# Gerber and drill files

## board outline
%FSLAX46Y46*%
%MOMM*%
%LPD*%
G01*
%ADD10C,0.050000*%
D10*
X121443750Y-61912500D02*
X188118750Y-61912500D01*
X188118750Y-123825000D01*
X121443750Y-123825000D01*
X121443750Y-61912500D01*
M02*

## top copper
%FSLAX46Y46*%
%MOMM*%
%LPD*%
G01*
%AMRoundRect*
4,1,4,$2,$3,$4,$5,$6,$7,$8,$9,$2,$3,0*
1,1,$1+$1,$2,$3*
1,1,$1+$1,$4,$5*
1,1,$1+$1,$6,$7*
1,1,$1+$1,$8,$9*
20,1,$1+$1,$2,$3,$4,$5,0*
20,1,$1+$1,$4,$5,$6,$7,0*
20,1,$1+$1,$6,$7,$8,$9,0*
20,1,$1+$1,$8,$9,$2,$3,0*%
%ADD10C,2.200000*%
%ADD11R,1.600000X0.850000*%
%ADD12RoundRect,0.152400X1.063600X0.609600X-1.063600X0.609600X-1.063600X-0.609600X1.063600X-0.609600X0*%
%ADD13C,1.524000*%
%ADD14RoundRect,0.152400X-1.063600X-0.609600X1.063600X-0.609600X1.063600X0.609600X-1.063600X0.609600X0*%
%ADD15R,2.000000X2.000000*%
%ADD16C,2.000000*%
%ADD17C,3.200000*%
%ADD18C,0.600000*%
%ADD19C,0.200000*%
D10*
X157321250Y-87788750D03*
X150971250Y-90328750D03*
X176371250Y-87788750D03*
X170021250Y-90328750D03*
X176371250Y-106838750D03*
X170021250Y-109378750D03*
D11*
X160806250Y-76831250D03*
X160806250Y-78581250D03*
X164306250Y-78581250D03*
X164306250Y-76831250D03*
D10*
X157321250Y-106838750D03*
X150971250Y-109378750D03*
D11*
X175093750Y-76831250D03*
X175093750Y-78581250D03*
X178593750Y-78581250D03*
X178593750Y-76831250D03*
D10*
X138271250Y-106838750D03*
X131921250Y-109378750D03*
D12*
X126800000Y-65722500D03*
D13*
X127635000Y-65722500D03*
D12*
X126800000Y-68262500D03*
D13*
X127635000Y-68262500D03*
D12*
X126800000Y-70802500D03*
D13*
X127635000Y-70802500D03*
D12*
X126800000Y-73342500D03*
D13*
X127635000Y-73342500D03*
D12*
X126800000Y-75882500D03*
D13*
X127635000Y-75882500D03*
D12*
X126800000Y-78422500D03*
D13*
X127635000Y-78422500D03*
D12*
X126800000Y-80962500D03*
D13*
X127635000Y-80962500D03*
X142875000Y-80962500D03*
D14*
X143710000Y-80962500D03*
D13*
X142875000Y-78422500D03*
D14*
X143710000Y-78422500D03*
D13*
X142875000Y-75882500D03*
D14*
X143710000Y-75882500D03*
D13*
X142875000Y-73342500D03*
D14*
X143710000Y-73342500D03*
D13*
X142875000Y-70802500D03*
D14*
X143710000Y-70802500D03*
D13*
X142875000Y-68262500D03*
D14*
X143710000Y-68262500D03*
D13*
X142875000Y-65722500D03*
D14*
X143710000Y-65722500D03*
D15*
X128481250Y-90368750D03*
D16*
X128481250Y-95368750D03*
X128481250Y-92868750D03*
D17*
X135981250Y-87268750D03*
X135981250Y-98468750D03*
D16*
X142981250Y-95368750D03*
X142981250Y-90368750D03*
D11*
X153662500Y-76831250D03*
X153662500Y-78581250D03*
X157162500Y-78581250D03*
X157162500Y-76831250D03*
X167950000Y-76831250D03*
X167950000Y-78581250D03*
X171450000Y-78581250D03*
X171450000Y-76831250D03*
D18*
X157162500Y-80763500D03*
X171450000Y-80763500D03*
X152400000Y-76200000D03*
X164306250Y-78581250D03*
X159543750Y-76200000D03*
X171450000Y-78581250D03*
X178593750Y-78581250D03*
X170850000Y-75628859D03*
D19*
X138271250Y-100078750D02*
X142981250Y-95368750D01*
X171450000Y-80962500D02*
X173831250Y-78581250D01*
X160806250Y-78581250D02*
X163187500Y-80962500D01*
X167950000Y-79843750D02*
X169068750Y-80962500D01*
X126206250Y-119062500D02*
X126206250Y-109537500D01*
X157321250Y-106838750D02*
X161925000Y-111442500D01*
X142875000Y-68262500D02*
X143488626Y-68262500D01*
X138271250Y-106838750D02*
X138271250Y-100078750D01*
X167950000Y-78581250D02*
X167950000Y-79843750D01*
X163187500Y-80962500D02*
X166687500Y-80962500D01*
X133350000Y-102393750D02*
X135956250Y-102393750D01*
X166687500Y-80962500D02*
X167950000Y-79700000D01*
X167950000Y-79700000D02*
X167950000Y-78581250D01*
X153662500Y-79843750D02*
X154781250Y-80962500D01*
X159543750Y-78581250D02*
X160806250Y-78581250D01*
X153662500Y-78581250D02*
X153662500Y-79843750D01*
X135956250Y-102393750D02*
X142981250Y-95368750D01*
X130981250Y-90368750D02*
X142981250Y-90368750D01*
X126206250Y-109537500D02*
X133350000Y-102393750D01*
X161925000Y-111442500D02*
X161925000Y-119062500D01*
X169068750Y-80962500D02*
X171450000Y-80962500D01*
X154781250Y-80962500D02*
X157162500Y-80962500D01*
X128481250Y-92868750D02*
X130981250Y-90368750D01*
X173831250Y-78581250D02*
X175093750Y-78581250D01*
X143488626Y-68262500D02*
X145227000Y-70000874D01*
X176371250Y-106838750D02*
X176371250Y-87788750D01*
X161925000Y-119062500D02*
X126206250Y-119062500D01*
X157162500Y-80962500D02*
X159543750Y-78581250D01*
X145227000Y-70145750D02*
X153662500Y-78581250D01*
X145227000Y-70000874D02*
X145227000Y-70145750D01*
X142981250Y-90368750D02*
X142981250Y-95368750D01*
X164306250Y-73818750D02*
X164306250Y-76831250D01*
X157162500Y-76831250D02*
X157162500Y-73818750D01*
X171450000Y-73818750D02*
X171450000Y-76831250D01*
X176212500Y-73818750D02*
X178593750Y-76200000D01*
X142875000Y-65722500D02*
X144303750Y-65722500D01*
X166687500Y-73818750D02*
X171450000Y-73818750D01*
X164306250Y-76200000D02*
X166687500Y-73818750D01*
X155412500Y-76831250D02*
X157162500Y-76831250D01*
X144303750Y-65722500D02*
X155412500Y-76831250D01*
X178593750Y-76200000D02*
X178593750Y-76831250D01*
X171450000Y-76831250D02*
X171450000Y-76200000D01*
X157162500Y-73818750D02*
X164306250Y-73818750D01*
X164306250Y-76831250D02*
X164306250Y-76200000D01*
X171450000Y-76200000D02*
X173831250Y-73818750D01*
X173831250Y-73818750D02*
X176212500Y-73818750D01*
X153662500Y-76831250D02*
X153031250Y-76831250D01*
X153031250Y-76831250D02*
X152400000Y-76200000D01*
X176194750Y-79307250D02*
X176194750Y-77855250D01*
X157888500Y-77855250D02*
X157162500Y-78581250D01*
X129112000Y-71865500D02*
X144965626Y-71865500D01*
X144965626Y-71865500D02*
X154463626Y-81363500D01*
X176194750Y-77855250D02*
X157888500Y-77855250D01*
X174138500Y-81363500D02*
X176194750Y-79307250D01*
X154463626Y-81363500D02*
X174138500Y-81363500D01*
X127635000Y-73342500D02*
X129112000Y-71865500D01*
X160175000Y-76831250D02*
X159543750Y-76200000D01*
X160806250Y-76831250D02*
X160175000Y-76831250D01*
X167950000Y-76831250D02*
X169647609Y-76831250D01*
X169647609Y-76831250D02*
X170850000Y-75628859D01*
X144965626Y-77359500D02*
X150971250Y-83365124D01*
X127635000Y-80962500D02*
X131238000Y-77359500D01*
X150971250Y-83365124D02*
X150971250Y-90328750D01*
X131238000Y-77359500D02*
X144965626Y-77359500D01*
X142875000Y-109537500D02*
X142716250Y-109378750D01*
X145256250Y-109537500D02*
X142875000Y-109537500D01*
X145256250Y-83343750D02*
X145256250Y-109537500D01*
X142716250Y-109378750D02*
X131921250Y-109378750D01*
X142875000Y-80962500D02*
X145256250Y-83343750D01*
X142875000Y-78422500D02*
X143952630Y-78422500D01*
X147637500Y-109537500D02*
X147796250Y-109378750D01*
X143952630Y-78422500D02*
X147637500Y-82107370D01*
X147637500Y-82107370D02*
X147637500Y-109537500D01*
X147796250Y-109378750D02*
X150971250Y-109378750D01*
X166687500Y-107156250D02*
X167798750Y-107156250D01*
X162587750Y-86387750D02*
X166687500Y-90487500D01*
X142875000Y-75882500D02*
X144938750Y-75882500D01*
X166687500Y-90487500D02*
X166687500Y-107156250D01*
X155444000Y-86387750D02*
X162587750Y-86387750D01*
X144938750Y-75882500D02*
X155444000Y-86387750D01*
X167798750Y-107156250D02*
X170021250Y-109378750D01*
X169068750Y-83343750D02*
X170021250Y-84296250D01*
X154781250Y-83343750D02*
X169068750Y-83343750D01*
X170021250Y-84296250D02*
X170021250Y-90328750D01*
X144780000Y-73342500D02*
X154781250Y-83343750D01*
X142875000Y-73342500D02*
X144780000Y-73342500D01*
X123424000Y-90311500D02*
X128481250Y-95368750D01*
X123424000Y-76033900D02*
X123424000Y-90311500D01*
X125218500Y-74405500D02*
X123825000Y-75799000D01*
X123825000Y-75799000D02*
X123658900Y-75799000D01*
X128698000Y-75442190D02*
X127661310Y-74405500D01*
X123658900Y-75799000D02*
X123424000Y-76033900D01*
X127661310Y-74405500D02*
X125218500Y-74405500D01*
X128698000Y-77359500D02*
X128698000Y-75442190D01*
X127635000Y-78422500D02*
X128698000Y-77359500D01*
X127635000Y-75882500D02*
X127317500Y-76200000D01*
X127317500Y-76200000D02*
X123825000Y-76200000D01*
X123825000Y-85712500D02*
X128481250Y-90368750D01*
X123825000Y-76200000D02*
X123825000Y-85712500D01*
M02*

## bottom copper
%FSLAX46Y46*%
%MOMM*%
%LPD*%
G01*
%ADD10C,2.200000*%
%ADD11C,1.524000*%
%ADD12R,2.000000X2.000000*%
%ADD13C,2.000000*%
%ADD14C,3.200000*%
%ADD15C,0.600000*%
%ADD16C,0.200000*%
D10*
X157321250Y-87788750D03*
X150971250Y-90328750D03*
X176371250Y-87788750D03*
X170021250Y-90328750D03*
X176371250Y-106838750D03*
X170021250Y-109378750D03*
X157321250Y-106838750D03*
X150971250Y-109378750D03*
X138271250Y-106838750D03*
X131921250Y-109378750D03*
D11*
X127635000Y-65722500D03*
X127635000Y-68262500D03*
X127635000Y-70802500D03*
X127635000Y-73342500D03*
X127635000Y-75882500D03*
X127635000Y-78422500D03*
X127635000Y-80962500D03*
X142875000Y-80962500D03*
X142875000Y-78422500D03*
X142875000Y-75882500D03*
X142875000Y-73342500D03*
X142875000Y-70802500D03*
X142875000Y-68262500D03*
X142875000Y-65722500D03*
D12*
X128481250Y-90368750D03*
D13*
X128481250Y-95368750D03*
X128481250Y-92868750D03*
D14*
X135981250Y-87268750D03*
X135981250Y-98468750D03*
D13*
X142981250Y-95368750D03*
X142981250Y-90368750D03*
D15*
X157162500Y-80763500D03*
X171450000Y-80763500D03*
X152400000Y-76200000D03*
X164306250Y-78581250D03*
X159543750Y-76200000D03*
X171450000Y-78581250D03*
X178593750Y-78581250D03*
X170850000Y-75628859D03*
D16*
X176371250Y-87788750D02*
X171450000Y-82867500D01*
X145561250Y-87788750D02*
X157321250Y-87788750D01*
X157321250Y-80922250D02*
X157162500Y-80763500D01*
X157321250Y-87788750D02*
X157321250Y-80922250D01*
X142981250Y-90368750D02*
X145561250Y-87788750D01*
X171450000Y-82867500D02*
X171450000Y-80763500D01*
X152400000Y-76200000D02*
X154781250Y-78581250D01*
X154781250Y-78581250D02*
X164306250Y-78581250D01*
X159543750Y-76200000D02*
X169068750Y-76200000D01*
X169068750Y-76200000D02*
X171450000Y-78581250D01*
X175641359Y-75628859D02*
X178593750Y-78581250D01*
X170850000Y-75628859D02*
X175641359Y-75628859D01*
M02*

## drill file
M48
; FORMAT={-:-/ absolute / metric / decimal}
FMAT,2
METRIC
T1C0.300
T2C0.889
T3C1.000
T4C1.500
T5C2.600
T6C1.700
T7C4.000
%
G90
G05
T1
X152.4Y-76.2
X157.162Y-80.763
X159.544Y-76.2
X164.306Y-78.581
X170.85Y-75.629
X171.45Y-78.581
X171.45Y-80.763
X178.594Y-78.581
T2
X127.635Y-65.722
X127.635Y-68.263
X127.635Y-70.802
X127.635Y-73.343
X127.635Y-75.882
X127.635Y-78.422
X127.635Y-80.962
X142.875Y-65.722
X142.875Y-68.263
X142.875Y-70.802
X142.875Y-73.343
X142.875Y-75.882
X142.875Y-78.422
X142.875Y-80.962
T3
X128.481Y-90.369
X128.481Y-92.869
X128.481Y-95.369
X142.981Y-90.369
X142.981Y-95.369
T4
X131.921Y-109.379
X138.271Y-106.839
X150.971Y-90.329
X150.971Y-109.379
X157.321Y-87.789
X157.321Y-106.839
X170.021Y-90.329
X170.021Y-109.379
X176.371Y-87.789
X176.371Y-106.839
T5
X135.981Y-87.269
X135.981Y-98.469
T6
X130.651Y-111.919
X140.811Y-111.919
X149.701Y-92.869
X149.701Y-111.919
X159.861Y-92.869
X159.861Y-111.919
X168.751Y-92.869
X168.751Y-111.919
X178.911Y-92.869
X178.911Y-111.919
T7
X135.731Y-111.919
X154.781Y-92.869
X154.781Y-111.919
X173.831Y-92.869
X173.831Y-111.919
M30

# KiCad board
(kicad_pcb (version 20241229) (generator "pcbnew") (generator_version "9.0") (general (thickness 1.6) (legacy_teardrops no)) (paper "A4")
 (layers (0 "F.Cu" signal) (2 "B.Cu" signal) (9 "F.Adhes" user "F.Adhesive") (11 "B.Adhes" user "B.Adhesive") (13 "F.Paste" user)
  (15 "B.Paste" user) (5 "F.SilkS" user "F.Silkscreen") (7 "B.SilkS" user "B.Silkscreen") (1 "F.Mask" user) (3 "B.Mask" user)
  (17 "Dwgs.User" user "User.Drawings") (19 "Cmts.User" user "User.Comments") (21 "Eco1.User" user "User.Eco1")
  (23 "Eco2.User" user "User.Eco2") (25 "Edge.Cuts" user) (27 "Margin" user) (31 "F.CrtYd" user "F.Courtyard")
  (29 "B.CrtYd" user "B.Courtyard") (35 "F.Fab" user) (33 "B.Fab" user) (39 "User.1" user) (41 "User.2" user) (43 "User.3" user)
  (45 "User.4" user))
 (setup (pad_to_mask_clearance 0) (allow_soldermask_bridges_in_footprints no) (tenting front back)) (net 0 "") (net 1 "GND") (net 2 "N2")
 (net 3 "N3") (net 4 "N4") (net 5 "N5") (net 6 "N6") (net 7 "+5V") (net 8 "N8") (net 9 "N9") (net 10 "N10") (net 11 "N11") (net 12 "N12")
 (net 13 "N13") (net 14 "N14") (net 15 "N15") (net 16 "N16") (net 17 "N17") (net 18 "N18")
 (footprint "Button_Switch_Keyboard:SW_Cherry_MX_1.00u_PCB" (layer "F.Cu") (at 157.32125 87.78875)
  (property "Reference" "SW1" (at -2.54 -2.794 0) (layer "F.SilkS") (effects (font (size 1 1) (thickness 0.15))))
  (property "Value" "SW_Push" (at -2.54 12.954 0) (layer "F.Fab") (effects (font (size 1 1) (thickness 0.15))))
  (pad "" np_thru_hole circle (at -7.62 5.08) (size 1.7 1.7) (drill 1.7) (layers "*.Cu" "*.Mask"))
  (pad "" np_thru_hole circle (at -2.54 5.08) (size 4 4) (drill 4) (layers "*.Cu" "*.Mask"))
  (pad "" np_thru_hole circle (at 2.54 5.08) (size 1.7 1.7) (drill 1.7) (layers "*.Cu" "*.Mask"))
  (pad "1" thru_hole circle (at 0 0) (size 2.2 2.2) (drill 1.5) (layers "*.Cu" "*.Mask") (remove_unused_layers no) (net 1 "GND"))
  (pad "2" thru_hole circle (at -6.35 2.54) (size 2.2 2.2) (drill 1.5) (layers "*.Cu" "*.Mask") (remove_unused_layers no) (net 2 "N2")))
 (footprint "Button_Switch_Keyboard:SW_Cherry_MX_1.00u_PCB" (layer "F.Cu") (at 176.37125 87.78875)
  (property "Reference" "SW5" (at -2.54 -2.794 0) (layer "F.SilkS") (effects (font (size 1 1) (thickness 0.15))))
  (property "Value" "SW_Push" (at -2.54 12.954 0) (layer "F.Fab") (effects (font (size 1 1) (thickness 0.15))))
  (pad "" np_thru_hole circle (at -7.62 5.08) (size 1.7 1.7) (drill 1.7) (layers "*.Cu" "*.Mask"))
  (pad "" np_thru_hole circle (at -2.54 5.08) (size 4 4) (drill 4) (layers "*.Cu" "*.Mask"))
  (pad "" np_thru_hole circle (at 2.54 5.08) (size 1.7 1.7) (drill 1.7) (layers "*.Cu" "*.Mask"))
  (pad "1" thru_hole circle (at 0 0) (size 2.2 2.2) (drill 1.5) (layers "*.Cu" "*.Mask") (remove_unused_layers no) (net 1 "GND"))
  (pad "2" thru_hole circle (at -6.35 2.54) (size 2.2 2.2) (drill 1.5) (layers "*.Cu" "*.Mask") (remove_unused_layers no) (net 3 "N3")))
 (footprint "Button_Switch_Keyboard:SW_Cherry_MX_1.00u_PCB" (layer "F.Cu") (at 176.37125 106.83875)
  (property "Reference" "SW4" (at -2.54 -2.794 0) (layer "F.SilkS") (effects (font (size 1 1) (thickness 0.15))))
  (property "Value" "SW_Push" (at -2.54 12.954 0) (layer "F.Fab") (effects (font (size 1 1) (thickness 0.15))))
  (pad "" np_thru_hole circle (at -7.62 5.08) (size 1.7 1.7) (drill 1.7) (layers "*.Cu" "*.Mask"))
  (pad "" np_thru_hole circle (at -2.54 5.08) (size 4 4) (drill 4) (layers "*.Cu" "*.Mask"))
  (pad "" np_thru_hole circle (at 2.54 5.08) (size 1.7 1.7) (drill 1.7) (layers "*.Cu" "*.Mask"))
  (pad "1" thru_hole circle (at 0 0) (size 2.2 2.2) (drill 1.5) (layers "*.Cu" "*.Mask") (remove_unused_layers no) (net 1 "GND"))
  (pad "2" thru_hole circle (at -6.35 2.54) (size 2.2 2.2) (drill 1.5) (layers "*.Cu" "*.Mask") (remove_unused_layers no) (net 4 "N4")))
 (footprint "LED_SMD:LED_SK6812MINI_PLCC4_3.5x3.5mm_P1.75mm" (layer "F.Cu") (at 162.55625 77.70625)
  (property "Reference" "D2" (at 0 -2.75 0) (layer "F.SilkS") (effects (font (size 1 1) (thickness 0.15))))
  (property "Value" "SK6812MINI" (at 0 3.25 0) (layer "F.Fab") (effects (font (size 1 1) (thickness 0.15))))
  (pad "1" smd rect (at -1.75 -0.875) (size 1.6 0.85) (layers "F.Cu" "F.Mask" "F.Paste") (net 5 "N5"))
  (pad "2" smd rect (at -1.75 0.875) (size 1.6 0.85) (layers "F.Cu" "F.Mask" "F.Paste") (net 1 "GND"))
  (pad "3" smd rect (at 1.75 0.875) (size 1.6 0.85) (layers "F.Cu" "F.Mask" "F.Paste") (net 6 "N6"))
  (pad "4" smd rect (at 1.75 -0.875) (size 1.6 0.85) (layers "F.Cu" "F.Mask" "F.Paste") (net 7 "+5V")))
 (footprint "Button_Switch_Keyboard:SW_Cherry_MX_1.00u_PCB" (layer "F.Cu") (at 157.32125 106.83875)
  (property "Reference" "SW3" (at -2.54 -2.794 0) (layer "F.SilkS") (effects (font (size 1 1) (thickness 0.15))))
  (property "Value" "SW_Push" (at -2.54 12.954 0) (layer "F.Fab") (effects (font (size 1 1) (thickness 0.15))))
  (pad "" np_thru_hole circle (at -7.62 5.08) (size 1.7 1.7) (drill 1.7) (layers "*.Cu" "*.Mask"))
  (pad "" np_thru_hole circle (at -2.54 5.08) (size 4 4) (drill 4) (layers "*.Cu" "*.Mask"))
  (pad "" np_thru_hole circle (at 2.54 5.08) (size 1.7 1.7) (drill 1.7) (layers "*.Cu" "*.Mask"))
  (pad "1" thru_hole circle (at 0 0) (size 2.2 2.2) (drill 1.5) (layers "*.Cu" "*.Mask") (remove_unused_layers no) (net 1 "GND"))
  (pad "2" thru_hole circle (at -6.35 2.54) (size 2.2 2.2) (drill 1.5) (layers "*.Cu" "*.Mask") (remove_unused_layers no) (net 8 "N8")))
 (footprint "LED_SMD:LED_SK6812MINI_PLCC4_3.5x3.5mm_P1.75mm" (layer "F.Cu") (at 176.84375 77.70625)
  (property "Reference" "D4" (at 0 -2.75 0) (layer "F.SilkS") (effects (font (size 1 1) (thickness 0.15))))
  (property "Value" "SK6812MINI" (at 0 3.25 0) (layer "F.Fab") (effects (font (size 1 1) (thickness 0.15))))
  (pad "1" smd rect (at -1.75 -0.875) (size 1.6 0.85) (layers "F.Cu" "F.Mask" "F.Paste") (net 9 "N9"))
  (pad "2" smd rect (at -1.75 0.875) (size 1.6 0.85) (layers "F.Cu" "F.Mask" "F.Paste") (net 1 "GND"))
  (pad "3" smd rect (at 1.75 0.875) (size 1.6 0.85) (layers "F.Cu" "F.Mask" "F.Paste") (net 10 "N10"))
  (pad "4" smd rect (at 1.75 -0.875) (size 1.6 0.85) (layers "F.Cu" "F.Mask" "F.Paste") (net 7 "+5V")))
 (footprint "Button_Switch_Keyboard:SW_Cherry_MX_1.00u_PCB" (layer "F.Cu") (at 138.27125 106.83875)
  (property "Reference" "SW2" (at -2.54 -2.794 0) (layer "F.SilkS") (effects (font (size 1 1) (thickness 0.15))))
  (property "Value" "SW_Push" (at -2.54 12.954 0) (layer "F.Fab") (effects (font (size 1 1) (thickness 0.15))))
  (pad "" np_thru_hole circle (at -7.62 5.08) (size 1.7 1.7) (drill 1.7) (layers "*.Cu" "*.Mask"))
  (pad "" np_thru_hole circle (at -2.54 5.08) (size 4 4) (drill 4) (layers "*.Cu" "*.Mask"))
  (pad "" np_thru_hole circle (at 2.54 5.08) (size 1.7 1.7) (drill 1.7) (layers "*.Cu" "*.Mask"))
  (pad "1" thru_hole circle (at 0 0) (size 2.2 2.2) (drill 1.5) (layers "*.Cu" "*.Mask") (remove_unused_layers no) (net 1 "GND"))
  (pad "2" thru_hole circle (at -6.35 2.54) (size 2.2 2.2) (drill 1.5) (layers "*.Cu" "*.Mask") (remove_unused_layers no) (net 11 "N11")))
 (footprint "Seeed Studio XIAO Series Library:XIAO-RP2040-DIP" (layer "F.Cu") (at 135.255 73.3425)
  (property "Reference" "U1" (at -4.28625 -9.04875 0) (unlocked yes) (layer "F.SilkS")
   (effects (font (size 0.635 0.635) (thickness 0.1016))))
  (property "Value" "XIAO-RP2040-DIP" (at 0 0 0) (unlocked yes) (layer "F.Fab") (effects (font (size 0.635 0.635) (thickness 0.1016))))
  (pad "1" smd roundrect (at -8.455 -7.62 180) (size 2.432 1.524) (layers "F.Cu" "F.Mask") (roundrect_rratio 0.1) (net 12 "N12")
   (thermal_bridge_angle 45))
  (pad "1" thru_hole circle (at -7.62 -7.62 180) (size 1.524 1.524) (drill 0.889) (layers "*.Cu" "*.Mask") (remove_unused_layers no)
   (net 12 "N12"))
  (pad "2" smd roundrect (at -8.455 -5.08 180) (size 2.432 1.524) (layers "F.Cu" "F.Mask") (roundrect_rratio 0.1) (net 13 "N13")
   (thermal_bridge_angle 45))
  (pad "2" thru_hole circle (at -7.62 -5.08 180) (size 1.524 1.524) (drill 0.889) (layers "*.Cu" "*.Mask") (remove_unused_layers no)
   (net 13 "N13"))
  (pad "3" smd roundrect (at -8.455 -2.54 180) (size 2.432 1.524) (layers "F.Cu" "F.Mask") (roundrect_rratio 0.1) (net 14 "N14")
   (thermal_bridge_angle 45))
  (pad "3" thru_hole circle (at -7.62 -2.54 180) (size 1.524 1.524) (drill 0.889) (layers "*.Cu" "*.Mask") (remove_unused_layers no)
   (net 14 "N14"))
  (pad "4" smd roundrect (at -8.455 0 180) (size 2.432 1.524) (layers "F.Cu" "F.Mask") (roundrect_rratio 0.1) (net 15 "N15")
   (thermal_bridge_angle 45))
  (pad "4" thru_hole circle (at -7.62 0 180) (size 1.524 1.524) (drill 0.889) (layers "*.Cu" "*.Mask") (remove_unused_layers no)
   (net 15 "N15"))
  (pad "5" smd roundrect (at -8.455 2.54 180) (size 2.432 1.524) (layers "F.Cu" "F.Mask") (roundrect_rratio 0.1) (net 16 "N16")
   (thermal_bridge_angle 45))
  (pad "5" thru_hole circle (at -7.62 2.54 180) (size 1.524 1.524) (drill 0.889) (layers "*.Cu" "*.Mask") (remove_unused_layers no)
   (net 16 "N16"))
  (pad "6" smd roundrect (at -8.455 5.08 180) (size 2.432 1.524) (layers "F.Cu" "F.Mask") (roundrect_rratio 0.1) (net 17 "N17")
   (thermal_bridge_angle 45))
  (pad "6" thru_hole circle (at -7.62 5.08 180) (size 1.524 1.524) (drill 0.889) (layers "*.Cu" "*.Mask") (remove_unused_layers no)
   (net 17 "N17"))
  (pad "7" smd roundrect (at -8.455 7.62 180) (size 2.432 1.524) (layers "F.Cu" "F.Mask") (roundrect_rratio 0.1) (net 2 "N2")
   (thermal_bridge_angle 45))
  (pad "7" thru_hole circle (at -7.62 7.62 180) (size 1.524 1.524) (drill 0.889) (layers "*.Cu" "*.Mask") (remove_unused_layers no)
   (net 2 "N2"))
  (pad "8" thru_hole circle (at 7.62 7.62) (size 1.524 1.524) (drill 0.889) (layers "*.Cu" "*.Mask") (remove_unused_layers no)
   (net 11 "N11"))
  (pad "8" smd roundrect (at 8.455 7.62) (size 2.432 1.524) (layers "F.Cu" "F.Mask") (roundrect_rratio 0.1) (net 11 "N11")
   (thermal_bridge_angle 45))
  (pad "9" thru_hole circle (at 7.62 5.08) (size 1.524 1.524) (drill 0.889) (layers "*.Cu" "*.Mask") (remove_unused_layers no) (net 8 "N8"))
  (pad "9" smd roundrect (at 8.455 5.08) (size 2.432 1.524) (layers "F.Cu" "F.Mask") (roundrect_rratio 0.1) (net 8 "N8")
   (thermal_bridge_angle 45))
  (pad "10" thru_hole circle (at 7.62 2.54) (size 1.524 1.524) (drill 0.889) (layers "*.Cu" "*.Mask") (remove_unused_layers no) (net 4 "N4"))
  (pad "10" smd roundrect (at 8.455 2.54) (size 2.432 1.524) (layers "F.Cu" "F.Mask") (roundrect_rratio 0.1) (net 4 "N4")
   (thermal_bridge_angle 45))
  (pad "11" thru_hole circle (at 7.62 0) (size 1.524 1.524) (drill 0.889) (layers "*.Cu" "*.Mask") (remove_unused_layers no) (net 3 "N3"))
  (pad "11" smd roundrect (at 8.455 0) (size 2.432 1.524) (layers "F.Cu" "F.Mask") (roundrect_rratio 0.1) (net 3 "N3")
   (thermal_bridge_angle 45))
  (pad "12" thru_hole circle (at 7.62 -2.54) (size 1.524 1.524) (drill 0.889) (layers "*.Cu" "*.Mask") (remove_unused_layers no)
   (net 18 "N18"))
  (pad "12" smd roundrect (at 8.455 -2.54) (size 2.432 1.524) (layers "F.Cu" "F.Mask") (roundrect_rratio 0.1) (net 18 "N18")
   (thermal_bridge_angle 45))
  (pad "13" thru_hole circle (at 7.62 -5.08) (size 1.524 1.524) (drill 0.889) (layers "*.Cu" "*.Mask") (remove_unused_layers no)
   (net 1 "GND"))
  (pad "13" smd roundrect (at 8.455 -5.08) (size 2.432 1.524) (layers "F.Cu" "F.Mask") (roundrect_rratio 0.1) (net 1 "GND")
   (thermal_bridge_angle 45))
  (pad "14" thru_hole circle (at 7.62 -7.62) (size 1.524 1.524) (drill 0.889) (layers "*.Cu" "*.Mask") (remove_unused_layers no)
   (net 7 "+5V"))
  (pad "14" smd roundrect (at 8.455 -7.62) (size 2.432 1.524) (layers "F.Cu" "F.Mask") (roundrect_rratio 0.1) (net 7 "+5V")
   (thermal_bridge_angle 45)))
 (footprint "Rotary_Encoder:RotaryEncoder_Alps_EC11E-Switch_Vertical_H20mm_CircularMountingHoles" (layer "F.Cu") (at 128.48125 90.36875)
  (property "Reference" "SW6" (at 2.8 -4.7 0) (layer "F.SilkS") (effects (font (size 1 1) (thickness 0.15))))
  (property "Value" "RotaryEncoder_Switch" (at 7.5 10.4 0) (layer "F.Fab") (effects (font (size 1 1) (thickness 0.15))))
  (pad "A" thru_hole rect (at 0 0) (size 2 2) (drill 1) (layers "*.Cu" "*.Mask") (remove_unused_layers no) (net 16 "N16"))
  (pad "B" thru_hole circle (at 0 5) (size 2 2) (drill 1) (layers "*.Cu" "*.Mask") (remove_unused_layers no) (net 17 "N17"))
  (pad "C" thru_hole circle (at 0 2.5) (size 2 2) (drill 1) (layers "*.Cu" "*.Mask") (remove_unused_layers no) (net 1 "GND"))
  (pad "MP" thru_hole circle (at 7.5 -3.1) (size 3.2 3.2) (drill 2.6) (layers "*.Cu" "*.Mask") (remove_unused_layers no))
  (pad "MP" thru_hole circle (at 7.5 8.1) (size 3.2 3.2) (drill 2.6) (layers "*.Cu" "*.Mask") (remove_unused_layers no))
  (pad "S1" thru_hole circle (at 14.5 5) (size 2 2) (drill 1) (layers "*.Cu" "*.Mask") (remove_unused_layers no) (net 1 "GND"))
  (pad "S2" thru_hole circle (at 14.5 0) (size 2 2) (drill 1) (layers "*.Cu" "*.Mask") (remove_unused_layers no) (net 1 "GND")))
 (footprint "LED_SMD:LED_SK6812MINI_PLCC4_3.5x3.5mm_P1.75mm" (layer "F.Cu") (at 155.4125 77.70625)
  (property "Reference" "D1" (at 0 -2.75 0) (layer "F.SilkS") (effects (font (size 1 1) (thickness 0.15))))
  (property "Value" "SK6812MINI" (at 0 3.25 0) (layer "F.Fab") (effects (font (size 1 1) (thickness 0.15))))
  (pad "1" smd rect (at -1.75 -0.875) (size 1.6 0.85) (layers "F.Cu" "F.Mask" "F.Paste") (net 6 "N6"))
  (pad "2" smd rect (at -1.75 0.875) (size 1.6 0.85) (layers "F.Cu" "F.Mask" "F.Paste") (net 1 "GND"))
  (pad "3" smd rect (at 1.75 0.875) (size 1.6 0.85) (layers "F.Cu" "F.Mask" "F.Paste") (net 15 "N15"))
  (pad "4" smd rect (at 1.75 -0.875) (size 1.6 0.85) (layers "F.Cu" "F.Mask" "F.Paste") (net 7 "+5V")))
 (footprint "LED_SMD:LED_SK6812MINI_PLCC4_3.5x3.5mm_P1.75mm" (layer "F.Cu") (at 169.7 77.70625)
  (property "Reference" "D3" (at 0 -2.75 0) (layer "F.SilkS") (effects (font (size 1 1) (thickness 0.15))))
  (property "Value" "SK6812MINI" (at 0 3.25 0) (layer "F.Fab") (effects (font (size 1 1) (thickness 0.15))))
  (pad "1" smd rect (at -1.75 -0.875) (size 1.6 0.85) (layers "F.Cu" "F.Mask" "F.Paste") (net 10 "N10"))
  (pad "2" smd rect (at -1.75 0.875) (size 1.6 0.85) (layers "F.Cu" "F.Mask" "F.Paste") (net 1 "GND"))
  (pad "3" smd rect (at 1.75 0.875) (size 1.6 0.85) (layers "F.Cu" "F.Mask" "F.Paste") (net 5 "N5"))
  (pad "4" smd rect (at 1.75 -0.875) (size 1.6 0.85) (layers "F.Cu" "F.Mask" "F.Paste") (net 7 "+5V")))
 (gr_rect (start 121.44375 61.9125) (end 188.11875 123.825) (stroke (width 0.05) (type default)) (fill no) (layer "Edge.Cuts"))
 (segment (start 138.27125 100.07875) (end 142.98125 95.36875) (width 0.2) (layer "F.Cu") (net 1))
 (segment (start 171.45 80.9625) (end 173.83125 78.58125) (width 0.2) (layer "F.Cu") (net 1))
 (segment (start 160.80625 78.58125) (end 163.1875 80.9625) (width 0.2) (layer "F.Cu") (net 1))
 (segment (start 167.95 79.84375) (end 169.06875 80.9625) (width 0.2) (layer "F.Cu") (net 1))
 (segment (start 126.20625 119.0625) (end 126.20625 109.5375) (width 0.2) (layer "F.Cu") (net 1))
 (segment (start 157.32125 106.83875) (end 161.925 111.4425) (width 0.2) (layer "F.Cu") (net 1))
 (segment (start 142.875 68.2625) (end 143.488626 68.2625) (width 0.2) (layer "F.Cu") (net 1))
 (segment (start 138.27125 106.83875) (end 138.27125 100.07875) (width 0.2) (layer "F.Cu") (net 1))
 (segment (start 167.95 78.58125) (end 167.95 79.84375) (width 0.2) (layer "F.Cu") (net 1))
 (segment (start 163.1875 80.9625) (end 166.6875 80.9625) (width 0.2) (layer "F.Cu") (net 1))
 (segment (start 133.35 102.39375) (end 135.95625 102.39375) (width 0.2) (layer "F.Cu") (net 1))
 (segment (start 166.6875 80.9625) (end 167.95 79.7) (width 0.2) (layer "F.Cu") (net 1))
 (segment (start 167.95 79.7) (end 167.95 78.58125) (width 0.2) (layer "F.Cu") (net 1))
 (segment (start 153.6625 79.84375) (end 154.78125 80.9625) (width 0.2) (layer "F.Cu") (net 1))
 (segment (start 159.54375 78.58125) (end 160.80625 78.58125) (width 0.2) (layer "F.Cu") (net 1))
 (segment (start 153.6625 78.58125) (end 153.6625 79.84375) (width 0.2) (layer "F.Cu") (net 1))
 (segment (start 135.95625 102.39375) (end 142.98125 95.36875) (width 0.2) (layer "F.Cu") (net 1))
 (segment (start 130.98125 90.36875) (end 142.98125 90.36875) (width 0.2) (layer "F.Cu") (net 1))
 (segment (start 126.20625 109.5375) (end 133.35 102.39375) (width 0.2) (layer "F.Cu") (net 1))
 (segment (start 161.925 111.4425) (end 161.925 119.0625) (width 0.2) (layer "F.Cu") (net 1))
 (segment (start 169.06875 80.9625) (end 171.45 80.9625) (width 0.2) (layer "F.Cu") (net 1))
 (segment (start 154.78125 80.9625) (end 157.1625 80.9625) (width 0.2) (layer "F.Cu") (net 1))
 (segment (start 128.48125 92.86875) (end 130.98125 90.36875) (width 0.2) (layer "F.Cu") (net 1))
 (segment (start 173.83125 78.58125) (end 175.09375 78.58125) (width 0.2) (layer "F.Cu") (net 1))
 (segment (start 143.488626 68.2625) (end 145.227 70.000874) (width 0.2) (layer "F.Cu") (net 1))
 (segment (start 176.37125 106.83875) (end 176.37125 87.78875) (width 0.2) (layer "F.Cu") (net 1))
 (segment (start 161.925 119.0625) (end 126.20625 119.0625) (width 0.2) (layer "F.Cu") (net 1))
 (segment (start 157.1625 80.9625) (end 159.54375 78.58125) (width 0.2) (layer "F.Cu") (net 1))
 (segment (start 145.227 70.14575) (end 153.6625 78.58125) (width 0.2) (layer "F.Cu") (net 1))
 (segment (start 145.227 70.000874) (end 145.227 70.14575) (width 0.2) (layer "F.Cu") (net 1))
 (segment (start 142.98125 90.36875) (end 142.98125 95.36875) (width 0.2) (layer "F.Cu") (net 1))
 (via (at 157.1625 80.7635) (size 0.6) (drill 0.3) (layers "F.Cu" "B.Cu") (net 1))
 (via (at 171.45 80.7635) (size 0.6) (drill 0.3) (layers "F.Cu" "B.Cu") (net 1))
 (segment (start 176.37125 87.78875) (end 171.45 82.8675) (width 0.2) (layer "B.Cu") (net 1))
 (segment (start 145.56125 87.78875) (end 157.32125 87.78875) (width 0.2) (layer "B.Cu") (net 1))
 (segment (start 157.32125 80.92225) (end 157.1625 80.7635) (width 0.2) (layer "B.Cu") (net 1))
 (segment (start 157.32125 87.78875) (end 157.32125 80.92225) (width 0.2) (layer "B.Cu") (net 1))
 (segment (start 142.98125 90.36875) (end 145.56125 87.78875) (width 0.2) (layer "B.Cu") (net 1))
 (segment (start 171.45 82.8675) (end 171.45 80.7635) (width 0.2) (layer "B.Cu") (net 1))
 (segment (start 164.30625 73.81875) (end 164.30625 76.83125) (width 0.2) (layer "F.Cu") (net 7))
 (segment (start 157.1625 76.83125) (end 157.1625 73.81875) (width 0.2) (layer "F.Cu") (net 7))
 (segment (start 171.45 73.81875) (end 171.45 76.83125) (width 0.2) (layer "F.Cu") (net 7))
 (segment (start 176.2125 73.81875) (end 178.59375 76.2) (width 0.2) (layer "F.Cu") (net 7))
 (segment (start 142.875 65.7225) (end 144.30375 65.7225) (width 0.2) (layer "F.Cu") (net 7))
 (segment (start 166.6875 73.81875) (end 171.45 73.81875) (width 0.2) (layer "F.Cu") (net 7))
 (segment (start 164.30625 76.2) (end 166.6875 73.81875) (width 0.2) (layer "F.Cu") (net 7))
 (segment (start 155.4125 76.83125) (end 157.1625 76.83125) (width 0.2) (layer "F.Cu") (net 7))
 (segment (start 144.30375 65.7225) (end 155.4125 76.83125) (width 0.2) (layer "F.Cu") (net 7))
 (segment (start 178.59375 76.2) (end 178.59375 76.83125) (width 0.2) (layer "F.Cu") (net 7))
 (segment (start 171.45 76.83125) (end 171.45 76.2) (width 0.2) (layer "F.Cu") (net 7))
 (segment (start 157.1625 73.81875) (end 164.30625 73.81875) (width 0.2) (layer "F.Cu") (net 7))
 (segment (start 164.30625 76.83125) (end 164.30625 76.2) (width 0.2) (layer "F.Cu") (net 7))
 (segment (start 171.45 76.2) (end 173.83125 73.81875) (width 0.2) (layer "F.Cu") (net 7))
 (segment (start 173.83125 73.81875) (end 176.2125 73.81875) (width 0.2) (layer "F.Cu") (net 7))
 (segment (start 153.6625 76.83125) (end 153.03125 76.83125) (width 0.2) (layer "F.Cu") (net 6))
 (segment (start 153.03125 76.83125) (end 152.4 76.2) (width 0.2) (layer "F.Cu") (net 6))
 (via (at 152.4 76.2) (size 0.6) (drill 0.3) (layers "F.Cu" "B.Cu") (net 6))
 (via (at 164.30625 78.58125) (size 0.6) (drill 0.3) (layers "F.Cu" "B.Cu") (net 6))
 (segment (start 152.4 76.2) (end 154.78125 78.58125) (width 0.2) (layer "B.Cu") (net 6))
 (segment (start 154.78125 78.58125) (end 164.30625 78.58125) (width 0.2) (layer "B.Cu") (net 6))
 (segment (start 176.19475 79.30725) (end 176.19475 77.85525) (width 0.2) (layer "F.Cu") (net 15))
 (segment (start 157.8885 77.85525) (end 157.1625 78.58125) (width 0.2) (layer "F.Cu") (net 15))
 (segment (start 129.112 71.8655) (end 144.965626 71.8655) (width 0.2) (layer "F.Cu") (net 15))
 (segment (start 144.965626 71.8655) (end 154.463626 81.3635) (width 0.2) (layer "F.Cu") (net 15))
 (segment (start 176.19475 77.85525) (end 157.8885 77.85525) (width 0.2) (layer "F.Cu") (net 15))
 (segment (start 174.1385 81.3635) (end 176.19475 79.30725) (width 0.2) (layer "F.Cu") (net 15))
 (segment (start 154.463626 81.3635) (end 174.1385 81.3635) (width 0.2) (layer "F.Cu") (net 15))
 (segment (start 127.635 73.3425) (end 129.112 71.8655) (width 0.2) (layer "F.Cu") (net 15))
 (segment (start 160.175 76.83125) (end 159.54375 76.2) (width 0.2) (layer "F.Cu") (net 5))
 (segment (start 160.80625 76.83125) (end 160.175 76.83125) (width 0.2) (layer "F.Cu") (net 5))
 (via (at 159.54375 76.2) (size 0.6) (drill 0.3) (layers "F.Cu" "B.Cu") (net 5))
 (via (at 171.45 78.58125) (size 0.6) (drill 0.3) (layers "F.Cu" "B.Cu") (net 5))
 (segment (start 159.54375 76.2) (end 169.06875 76.2) (width 0.2) (layer "B.Cu") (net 5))
 (segment (start 169.06875 76.2) (end 171.45 78.58125) (width 0.2) (layer "B.Cu") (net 5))
 (segment (start 167.95 76.83125) (end 169.647609 76.83125) (width 0.2) (layer "F.Cu") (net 10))
 (segment (start 169.647609 76.83125) (end 170.85 75.628859) (width 0.2) (layer "F.Cu") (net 10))
 (via (at 178.59375 78.58125) (size 0.6) (drill 0.3) (layers "F.Cu" "B.Cu") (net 10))
 (via (at 170.85 75.628859) (size 0.6) (drill 0.3) (layers "F.Cu" "B.Cu") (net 10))
 (segment (start 175.641359 75.628859) (end 178.59375 78.58125) (width 0.2) (layer "B.Cu") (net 10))
 (segment (start 170.85 75.628859) (end 175.641359 75.628859) (width 0.2) (layer "B.Cu") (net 10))
 (segment (start 144.965626 77.3595) (end 150.97125 83.365124) (width 0.2) (layer "F.Cu") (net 2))
 (segment (start 127.635 80.9625) (end 131.238 77.3595) (width 0.2) (layer "F.Cu") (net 2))
 (segment (start 150.97125 83.365124) (end 150.97125 90.32875) (width 0.2) (layer "F.Cu") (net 2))
 (segment (start 131.238 77.3595) (end 144.965626 77.3595) (width 0.2) (layer "F.Cu") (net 2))
 (segment (start 142.875 109.5375) (end 142.71625 109.37875) (width 0.2) (layer "F.Cu") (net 11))
 (segment (start 145.25625 109.5375) (end 142.875 109.5375) (width 0.2) (layer "F.Cu") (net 11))
 (segment (start 145.25625 83.34375) (end 145.25625 109.5375) (width 0.2) (layer "F.Cu") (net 11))
 (segment (start 142.71625 109.37875) (end 131.92125 109.37875) (width 0.2) (layer "F.Cu") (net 11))
 (segment (start 142.875 80.9625) (end 145.25625 83.34375) (width 0.2) (layer "F.Cu") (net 11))
 (segment (start 142.875 78.4225) (end 143.95263 78.4225) (width 0.2) (layer "F.Cu") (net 8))
 (segment (start 147.6375 109.5375) (end 147.79625 109.37875) (width 0.2) (layer "F.Cu") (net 8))
 (segment (start 143.95263 78.4225) (end 147.6375 82.10737) (width 0.2) (layer "F.Cu") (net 8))
 (segment (start 147.6375 82.10737) (end 147.6375 109.5375) (width 0.2) (layer "F.Cu") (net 8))
 (segment (start 147.79625 109.37875) (end 150.97125 109.37875) (width 0.2) (layer "F.Cu") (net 8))
 (segment (start 166.6875 107.15625) (end 167.79875 107.15625) (width 0.2) (layer "F.Cu") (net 4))
 (segment (start 162.58775 86.38775) (end 166.6875 90.4875) (width 0.2) (layer "F.Cu") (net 4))
 (segment (start 142.875 75.8825) (end 144.93875 75.8825) (width 0.2) (layer "F.Cu") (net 4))
 (segment (start 166.6875 90.4875) (end 166.6875 107.15625) (width 0.2) (layer "F.Cu") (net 4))
 (segment (start 155.444 86.38775) (end 162.58775 86.38775) (width 0.2) (layer "F.Cu") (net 4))
 (segment (start 144.93875 75.8825) (end 155.444 86.38775) (width 0.2) (layer "F.Cu") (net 4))
 (segment (start 167.79875 107.15625) (end 170.02125 109.37875) (width 0.2) (layer "F.Cu") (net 4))
 (segment (start 169.06875 83.34375) (end 170.02125 84.29625) (width 0.2) (layer "F.Cu") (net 3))
 (segment (start 154.78125 83.34375) (end 169.06875 83.34375) (width 0.2) (layer "F.Cu") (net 3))
 (segment (start 170.02125 84.29625) (end 170.02125 90.32875) (width 0.2) (layer "F.Cu") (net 3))
 (segment (start 144.78 73.3425) (end 154.78125 83.34375) (width 0.2) (layer "F.Cu") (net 3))
 (segment (start 142.875 73.3425) (end 144.78 73.3425) (width 0.2) (layer "F.Cu") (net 3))
 (segment (start 123.424 90.3115) (end 128.48125 95.36875) (width 0.2) (layer "F.Cu") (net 17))
 (segment (start 123.424 76.0339) (end 123.424 90.3115) (width 0.2) (layer "F.Cu") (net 17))
 (segment (start 125.2185 74.4055) (end 123.825 75.799) (width 0.2) (layer "F.Cu") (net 17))
 (segment (start 123.825 75.799) (end 123.6589 75.799) (width 0.2) (layer "F.Cu") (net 17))
 (segment (start 128.698 75.44219) (end 127.66131 74.4055) (width 0.2) (layer "F.Cu") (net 17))
 (segment (start 123.6589 75.799) (end 123.424 76.0339) (width 0.2) (layer "F.Cu") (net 17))
 (segment (start 127.66131 74.4055) (end 125.2185 74.4055) (width 0.2) (layer "F.Cu") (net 17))
 (segment (start 128.698 77.3595) (end 128.698 75.44219) (width 0.2) (layer "F.Cu") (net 17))
 (segment (start 127.635 78.4225) (end 128.698 77.3595) (width 0.2) (layer "F.Cu") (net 17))
 (segment (start 127.635 75.8825) (end 127.3175 76.2) (width 0.2) (layer "F.Cu") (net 16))
 (segment (start 127.3175 76.2) (end 123.825 76.2) (width 0.2) (layer "F.Cu") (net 16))
 (segment (start 123.825 85.7125) (end 128.48125 90.36875) (width 0.2) (layer "F.Cu") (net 16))
 (segment (start 123.825 76.2) (end 123.825 85.7125) (width 0.2) (layer "F.Cu") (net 16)))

